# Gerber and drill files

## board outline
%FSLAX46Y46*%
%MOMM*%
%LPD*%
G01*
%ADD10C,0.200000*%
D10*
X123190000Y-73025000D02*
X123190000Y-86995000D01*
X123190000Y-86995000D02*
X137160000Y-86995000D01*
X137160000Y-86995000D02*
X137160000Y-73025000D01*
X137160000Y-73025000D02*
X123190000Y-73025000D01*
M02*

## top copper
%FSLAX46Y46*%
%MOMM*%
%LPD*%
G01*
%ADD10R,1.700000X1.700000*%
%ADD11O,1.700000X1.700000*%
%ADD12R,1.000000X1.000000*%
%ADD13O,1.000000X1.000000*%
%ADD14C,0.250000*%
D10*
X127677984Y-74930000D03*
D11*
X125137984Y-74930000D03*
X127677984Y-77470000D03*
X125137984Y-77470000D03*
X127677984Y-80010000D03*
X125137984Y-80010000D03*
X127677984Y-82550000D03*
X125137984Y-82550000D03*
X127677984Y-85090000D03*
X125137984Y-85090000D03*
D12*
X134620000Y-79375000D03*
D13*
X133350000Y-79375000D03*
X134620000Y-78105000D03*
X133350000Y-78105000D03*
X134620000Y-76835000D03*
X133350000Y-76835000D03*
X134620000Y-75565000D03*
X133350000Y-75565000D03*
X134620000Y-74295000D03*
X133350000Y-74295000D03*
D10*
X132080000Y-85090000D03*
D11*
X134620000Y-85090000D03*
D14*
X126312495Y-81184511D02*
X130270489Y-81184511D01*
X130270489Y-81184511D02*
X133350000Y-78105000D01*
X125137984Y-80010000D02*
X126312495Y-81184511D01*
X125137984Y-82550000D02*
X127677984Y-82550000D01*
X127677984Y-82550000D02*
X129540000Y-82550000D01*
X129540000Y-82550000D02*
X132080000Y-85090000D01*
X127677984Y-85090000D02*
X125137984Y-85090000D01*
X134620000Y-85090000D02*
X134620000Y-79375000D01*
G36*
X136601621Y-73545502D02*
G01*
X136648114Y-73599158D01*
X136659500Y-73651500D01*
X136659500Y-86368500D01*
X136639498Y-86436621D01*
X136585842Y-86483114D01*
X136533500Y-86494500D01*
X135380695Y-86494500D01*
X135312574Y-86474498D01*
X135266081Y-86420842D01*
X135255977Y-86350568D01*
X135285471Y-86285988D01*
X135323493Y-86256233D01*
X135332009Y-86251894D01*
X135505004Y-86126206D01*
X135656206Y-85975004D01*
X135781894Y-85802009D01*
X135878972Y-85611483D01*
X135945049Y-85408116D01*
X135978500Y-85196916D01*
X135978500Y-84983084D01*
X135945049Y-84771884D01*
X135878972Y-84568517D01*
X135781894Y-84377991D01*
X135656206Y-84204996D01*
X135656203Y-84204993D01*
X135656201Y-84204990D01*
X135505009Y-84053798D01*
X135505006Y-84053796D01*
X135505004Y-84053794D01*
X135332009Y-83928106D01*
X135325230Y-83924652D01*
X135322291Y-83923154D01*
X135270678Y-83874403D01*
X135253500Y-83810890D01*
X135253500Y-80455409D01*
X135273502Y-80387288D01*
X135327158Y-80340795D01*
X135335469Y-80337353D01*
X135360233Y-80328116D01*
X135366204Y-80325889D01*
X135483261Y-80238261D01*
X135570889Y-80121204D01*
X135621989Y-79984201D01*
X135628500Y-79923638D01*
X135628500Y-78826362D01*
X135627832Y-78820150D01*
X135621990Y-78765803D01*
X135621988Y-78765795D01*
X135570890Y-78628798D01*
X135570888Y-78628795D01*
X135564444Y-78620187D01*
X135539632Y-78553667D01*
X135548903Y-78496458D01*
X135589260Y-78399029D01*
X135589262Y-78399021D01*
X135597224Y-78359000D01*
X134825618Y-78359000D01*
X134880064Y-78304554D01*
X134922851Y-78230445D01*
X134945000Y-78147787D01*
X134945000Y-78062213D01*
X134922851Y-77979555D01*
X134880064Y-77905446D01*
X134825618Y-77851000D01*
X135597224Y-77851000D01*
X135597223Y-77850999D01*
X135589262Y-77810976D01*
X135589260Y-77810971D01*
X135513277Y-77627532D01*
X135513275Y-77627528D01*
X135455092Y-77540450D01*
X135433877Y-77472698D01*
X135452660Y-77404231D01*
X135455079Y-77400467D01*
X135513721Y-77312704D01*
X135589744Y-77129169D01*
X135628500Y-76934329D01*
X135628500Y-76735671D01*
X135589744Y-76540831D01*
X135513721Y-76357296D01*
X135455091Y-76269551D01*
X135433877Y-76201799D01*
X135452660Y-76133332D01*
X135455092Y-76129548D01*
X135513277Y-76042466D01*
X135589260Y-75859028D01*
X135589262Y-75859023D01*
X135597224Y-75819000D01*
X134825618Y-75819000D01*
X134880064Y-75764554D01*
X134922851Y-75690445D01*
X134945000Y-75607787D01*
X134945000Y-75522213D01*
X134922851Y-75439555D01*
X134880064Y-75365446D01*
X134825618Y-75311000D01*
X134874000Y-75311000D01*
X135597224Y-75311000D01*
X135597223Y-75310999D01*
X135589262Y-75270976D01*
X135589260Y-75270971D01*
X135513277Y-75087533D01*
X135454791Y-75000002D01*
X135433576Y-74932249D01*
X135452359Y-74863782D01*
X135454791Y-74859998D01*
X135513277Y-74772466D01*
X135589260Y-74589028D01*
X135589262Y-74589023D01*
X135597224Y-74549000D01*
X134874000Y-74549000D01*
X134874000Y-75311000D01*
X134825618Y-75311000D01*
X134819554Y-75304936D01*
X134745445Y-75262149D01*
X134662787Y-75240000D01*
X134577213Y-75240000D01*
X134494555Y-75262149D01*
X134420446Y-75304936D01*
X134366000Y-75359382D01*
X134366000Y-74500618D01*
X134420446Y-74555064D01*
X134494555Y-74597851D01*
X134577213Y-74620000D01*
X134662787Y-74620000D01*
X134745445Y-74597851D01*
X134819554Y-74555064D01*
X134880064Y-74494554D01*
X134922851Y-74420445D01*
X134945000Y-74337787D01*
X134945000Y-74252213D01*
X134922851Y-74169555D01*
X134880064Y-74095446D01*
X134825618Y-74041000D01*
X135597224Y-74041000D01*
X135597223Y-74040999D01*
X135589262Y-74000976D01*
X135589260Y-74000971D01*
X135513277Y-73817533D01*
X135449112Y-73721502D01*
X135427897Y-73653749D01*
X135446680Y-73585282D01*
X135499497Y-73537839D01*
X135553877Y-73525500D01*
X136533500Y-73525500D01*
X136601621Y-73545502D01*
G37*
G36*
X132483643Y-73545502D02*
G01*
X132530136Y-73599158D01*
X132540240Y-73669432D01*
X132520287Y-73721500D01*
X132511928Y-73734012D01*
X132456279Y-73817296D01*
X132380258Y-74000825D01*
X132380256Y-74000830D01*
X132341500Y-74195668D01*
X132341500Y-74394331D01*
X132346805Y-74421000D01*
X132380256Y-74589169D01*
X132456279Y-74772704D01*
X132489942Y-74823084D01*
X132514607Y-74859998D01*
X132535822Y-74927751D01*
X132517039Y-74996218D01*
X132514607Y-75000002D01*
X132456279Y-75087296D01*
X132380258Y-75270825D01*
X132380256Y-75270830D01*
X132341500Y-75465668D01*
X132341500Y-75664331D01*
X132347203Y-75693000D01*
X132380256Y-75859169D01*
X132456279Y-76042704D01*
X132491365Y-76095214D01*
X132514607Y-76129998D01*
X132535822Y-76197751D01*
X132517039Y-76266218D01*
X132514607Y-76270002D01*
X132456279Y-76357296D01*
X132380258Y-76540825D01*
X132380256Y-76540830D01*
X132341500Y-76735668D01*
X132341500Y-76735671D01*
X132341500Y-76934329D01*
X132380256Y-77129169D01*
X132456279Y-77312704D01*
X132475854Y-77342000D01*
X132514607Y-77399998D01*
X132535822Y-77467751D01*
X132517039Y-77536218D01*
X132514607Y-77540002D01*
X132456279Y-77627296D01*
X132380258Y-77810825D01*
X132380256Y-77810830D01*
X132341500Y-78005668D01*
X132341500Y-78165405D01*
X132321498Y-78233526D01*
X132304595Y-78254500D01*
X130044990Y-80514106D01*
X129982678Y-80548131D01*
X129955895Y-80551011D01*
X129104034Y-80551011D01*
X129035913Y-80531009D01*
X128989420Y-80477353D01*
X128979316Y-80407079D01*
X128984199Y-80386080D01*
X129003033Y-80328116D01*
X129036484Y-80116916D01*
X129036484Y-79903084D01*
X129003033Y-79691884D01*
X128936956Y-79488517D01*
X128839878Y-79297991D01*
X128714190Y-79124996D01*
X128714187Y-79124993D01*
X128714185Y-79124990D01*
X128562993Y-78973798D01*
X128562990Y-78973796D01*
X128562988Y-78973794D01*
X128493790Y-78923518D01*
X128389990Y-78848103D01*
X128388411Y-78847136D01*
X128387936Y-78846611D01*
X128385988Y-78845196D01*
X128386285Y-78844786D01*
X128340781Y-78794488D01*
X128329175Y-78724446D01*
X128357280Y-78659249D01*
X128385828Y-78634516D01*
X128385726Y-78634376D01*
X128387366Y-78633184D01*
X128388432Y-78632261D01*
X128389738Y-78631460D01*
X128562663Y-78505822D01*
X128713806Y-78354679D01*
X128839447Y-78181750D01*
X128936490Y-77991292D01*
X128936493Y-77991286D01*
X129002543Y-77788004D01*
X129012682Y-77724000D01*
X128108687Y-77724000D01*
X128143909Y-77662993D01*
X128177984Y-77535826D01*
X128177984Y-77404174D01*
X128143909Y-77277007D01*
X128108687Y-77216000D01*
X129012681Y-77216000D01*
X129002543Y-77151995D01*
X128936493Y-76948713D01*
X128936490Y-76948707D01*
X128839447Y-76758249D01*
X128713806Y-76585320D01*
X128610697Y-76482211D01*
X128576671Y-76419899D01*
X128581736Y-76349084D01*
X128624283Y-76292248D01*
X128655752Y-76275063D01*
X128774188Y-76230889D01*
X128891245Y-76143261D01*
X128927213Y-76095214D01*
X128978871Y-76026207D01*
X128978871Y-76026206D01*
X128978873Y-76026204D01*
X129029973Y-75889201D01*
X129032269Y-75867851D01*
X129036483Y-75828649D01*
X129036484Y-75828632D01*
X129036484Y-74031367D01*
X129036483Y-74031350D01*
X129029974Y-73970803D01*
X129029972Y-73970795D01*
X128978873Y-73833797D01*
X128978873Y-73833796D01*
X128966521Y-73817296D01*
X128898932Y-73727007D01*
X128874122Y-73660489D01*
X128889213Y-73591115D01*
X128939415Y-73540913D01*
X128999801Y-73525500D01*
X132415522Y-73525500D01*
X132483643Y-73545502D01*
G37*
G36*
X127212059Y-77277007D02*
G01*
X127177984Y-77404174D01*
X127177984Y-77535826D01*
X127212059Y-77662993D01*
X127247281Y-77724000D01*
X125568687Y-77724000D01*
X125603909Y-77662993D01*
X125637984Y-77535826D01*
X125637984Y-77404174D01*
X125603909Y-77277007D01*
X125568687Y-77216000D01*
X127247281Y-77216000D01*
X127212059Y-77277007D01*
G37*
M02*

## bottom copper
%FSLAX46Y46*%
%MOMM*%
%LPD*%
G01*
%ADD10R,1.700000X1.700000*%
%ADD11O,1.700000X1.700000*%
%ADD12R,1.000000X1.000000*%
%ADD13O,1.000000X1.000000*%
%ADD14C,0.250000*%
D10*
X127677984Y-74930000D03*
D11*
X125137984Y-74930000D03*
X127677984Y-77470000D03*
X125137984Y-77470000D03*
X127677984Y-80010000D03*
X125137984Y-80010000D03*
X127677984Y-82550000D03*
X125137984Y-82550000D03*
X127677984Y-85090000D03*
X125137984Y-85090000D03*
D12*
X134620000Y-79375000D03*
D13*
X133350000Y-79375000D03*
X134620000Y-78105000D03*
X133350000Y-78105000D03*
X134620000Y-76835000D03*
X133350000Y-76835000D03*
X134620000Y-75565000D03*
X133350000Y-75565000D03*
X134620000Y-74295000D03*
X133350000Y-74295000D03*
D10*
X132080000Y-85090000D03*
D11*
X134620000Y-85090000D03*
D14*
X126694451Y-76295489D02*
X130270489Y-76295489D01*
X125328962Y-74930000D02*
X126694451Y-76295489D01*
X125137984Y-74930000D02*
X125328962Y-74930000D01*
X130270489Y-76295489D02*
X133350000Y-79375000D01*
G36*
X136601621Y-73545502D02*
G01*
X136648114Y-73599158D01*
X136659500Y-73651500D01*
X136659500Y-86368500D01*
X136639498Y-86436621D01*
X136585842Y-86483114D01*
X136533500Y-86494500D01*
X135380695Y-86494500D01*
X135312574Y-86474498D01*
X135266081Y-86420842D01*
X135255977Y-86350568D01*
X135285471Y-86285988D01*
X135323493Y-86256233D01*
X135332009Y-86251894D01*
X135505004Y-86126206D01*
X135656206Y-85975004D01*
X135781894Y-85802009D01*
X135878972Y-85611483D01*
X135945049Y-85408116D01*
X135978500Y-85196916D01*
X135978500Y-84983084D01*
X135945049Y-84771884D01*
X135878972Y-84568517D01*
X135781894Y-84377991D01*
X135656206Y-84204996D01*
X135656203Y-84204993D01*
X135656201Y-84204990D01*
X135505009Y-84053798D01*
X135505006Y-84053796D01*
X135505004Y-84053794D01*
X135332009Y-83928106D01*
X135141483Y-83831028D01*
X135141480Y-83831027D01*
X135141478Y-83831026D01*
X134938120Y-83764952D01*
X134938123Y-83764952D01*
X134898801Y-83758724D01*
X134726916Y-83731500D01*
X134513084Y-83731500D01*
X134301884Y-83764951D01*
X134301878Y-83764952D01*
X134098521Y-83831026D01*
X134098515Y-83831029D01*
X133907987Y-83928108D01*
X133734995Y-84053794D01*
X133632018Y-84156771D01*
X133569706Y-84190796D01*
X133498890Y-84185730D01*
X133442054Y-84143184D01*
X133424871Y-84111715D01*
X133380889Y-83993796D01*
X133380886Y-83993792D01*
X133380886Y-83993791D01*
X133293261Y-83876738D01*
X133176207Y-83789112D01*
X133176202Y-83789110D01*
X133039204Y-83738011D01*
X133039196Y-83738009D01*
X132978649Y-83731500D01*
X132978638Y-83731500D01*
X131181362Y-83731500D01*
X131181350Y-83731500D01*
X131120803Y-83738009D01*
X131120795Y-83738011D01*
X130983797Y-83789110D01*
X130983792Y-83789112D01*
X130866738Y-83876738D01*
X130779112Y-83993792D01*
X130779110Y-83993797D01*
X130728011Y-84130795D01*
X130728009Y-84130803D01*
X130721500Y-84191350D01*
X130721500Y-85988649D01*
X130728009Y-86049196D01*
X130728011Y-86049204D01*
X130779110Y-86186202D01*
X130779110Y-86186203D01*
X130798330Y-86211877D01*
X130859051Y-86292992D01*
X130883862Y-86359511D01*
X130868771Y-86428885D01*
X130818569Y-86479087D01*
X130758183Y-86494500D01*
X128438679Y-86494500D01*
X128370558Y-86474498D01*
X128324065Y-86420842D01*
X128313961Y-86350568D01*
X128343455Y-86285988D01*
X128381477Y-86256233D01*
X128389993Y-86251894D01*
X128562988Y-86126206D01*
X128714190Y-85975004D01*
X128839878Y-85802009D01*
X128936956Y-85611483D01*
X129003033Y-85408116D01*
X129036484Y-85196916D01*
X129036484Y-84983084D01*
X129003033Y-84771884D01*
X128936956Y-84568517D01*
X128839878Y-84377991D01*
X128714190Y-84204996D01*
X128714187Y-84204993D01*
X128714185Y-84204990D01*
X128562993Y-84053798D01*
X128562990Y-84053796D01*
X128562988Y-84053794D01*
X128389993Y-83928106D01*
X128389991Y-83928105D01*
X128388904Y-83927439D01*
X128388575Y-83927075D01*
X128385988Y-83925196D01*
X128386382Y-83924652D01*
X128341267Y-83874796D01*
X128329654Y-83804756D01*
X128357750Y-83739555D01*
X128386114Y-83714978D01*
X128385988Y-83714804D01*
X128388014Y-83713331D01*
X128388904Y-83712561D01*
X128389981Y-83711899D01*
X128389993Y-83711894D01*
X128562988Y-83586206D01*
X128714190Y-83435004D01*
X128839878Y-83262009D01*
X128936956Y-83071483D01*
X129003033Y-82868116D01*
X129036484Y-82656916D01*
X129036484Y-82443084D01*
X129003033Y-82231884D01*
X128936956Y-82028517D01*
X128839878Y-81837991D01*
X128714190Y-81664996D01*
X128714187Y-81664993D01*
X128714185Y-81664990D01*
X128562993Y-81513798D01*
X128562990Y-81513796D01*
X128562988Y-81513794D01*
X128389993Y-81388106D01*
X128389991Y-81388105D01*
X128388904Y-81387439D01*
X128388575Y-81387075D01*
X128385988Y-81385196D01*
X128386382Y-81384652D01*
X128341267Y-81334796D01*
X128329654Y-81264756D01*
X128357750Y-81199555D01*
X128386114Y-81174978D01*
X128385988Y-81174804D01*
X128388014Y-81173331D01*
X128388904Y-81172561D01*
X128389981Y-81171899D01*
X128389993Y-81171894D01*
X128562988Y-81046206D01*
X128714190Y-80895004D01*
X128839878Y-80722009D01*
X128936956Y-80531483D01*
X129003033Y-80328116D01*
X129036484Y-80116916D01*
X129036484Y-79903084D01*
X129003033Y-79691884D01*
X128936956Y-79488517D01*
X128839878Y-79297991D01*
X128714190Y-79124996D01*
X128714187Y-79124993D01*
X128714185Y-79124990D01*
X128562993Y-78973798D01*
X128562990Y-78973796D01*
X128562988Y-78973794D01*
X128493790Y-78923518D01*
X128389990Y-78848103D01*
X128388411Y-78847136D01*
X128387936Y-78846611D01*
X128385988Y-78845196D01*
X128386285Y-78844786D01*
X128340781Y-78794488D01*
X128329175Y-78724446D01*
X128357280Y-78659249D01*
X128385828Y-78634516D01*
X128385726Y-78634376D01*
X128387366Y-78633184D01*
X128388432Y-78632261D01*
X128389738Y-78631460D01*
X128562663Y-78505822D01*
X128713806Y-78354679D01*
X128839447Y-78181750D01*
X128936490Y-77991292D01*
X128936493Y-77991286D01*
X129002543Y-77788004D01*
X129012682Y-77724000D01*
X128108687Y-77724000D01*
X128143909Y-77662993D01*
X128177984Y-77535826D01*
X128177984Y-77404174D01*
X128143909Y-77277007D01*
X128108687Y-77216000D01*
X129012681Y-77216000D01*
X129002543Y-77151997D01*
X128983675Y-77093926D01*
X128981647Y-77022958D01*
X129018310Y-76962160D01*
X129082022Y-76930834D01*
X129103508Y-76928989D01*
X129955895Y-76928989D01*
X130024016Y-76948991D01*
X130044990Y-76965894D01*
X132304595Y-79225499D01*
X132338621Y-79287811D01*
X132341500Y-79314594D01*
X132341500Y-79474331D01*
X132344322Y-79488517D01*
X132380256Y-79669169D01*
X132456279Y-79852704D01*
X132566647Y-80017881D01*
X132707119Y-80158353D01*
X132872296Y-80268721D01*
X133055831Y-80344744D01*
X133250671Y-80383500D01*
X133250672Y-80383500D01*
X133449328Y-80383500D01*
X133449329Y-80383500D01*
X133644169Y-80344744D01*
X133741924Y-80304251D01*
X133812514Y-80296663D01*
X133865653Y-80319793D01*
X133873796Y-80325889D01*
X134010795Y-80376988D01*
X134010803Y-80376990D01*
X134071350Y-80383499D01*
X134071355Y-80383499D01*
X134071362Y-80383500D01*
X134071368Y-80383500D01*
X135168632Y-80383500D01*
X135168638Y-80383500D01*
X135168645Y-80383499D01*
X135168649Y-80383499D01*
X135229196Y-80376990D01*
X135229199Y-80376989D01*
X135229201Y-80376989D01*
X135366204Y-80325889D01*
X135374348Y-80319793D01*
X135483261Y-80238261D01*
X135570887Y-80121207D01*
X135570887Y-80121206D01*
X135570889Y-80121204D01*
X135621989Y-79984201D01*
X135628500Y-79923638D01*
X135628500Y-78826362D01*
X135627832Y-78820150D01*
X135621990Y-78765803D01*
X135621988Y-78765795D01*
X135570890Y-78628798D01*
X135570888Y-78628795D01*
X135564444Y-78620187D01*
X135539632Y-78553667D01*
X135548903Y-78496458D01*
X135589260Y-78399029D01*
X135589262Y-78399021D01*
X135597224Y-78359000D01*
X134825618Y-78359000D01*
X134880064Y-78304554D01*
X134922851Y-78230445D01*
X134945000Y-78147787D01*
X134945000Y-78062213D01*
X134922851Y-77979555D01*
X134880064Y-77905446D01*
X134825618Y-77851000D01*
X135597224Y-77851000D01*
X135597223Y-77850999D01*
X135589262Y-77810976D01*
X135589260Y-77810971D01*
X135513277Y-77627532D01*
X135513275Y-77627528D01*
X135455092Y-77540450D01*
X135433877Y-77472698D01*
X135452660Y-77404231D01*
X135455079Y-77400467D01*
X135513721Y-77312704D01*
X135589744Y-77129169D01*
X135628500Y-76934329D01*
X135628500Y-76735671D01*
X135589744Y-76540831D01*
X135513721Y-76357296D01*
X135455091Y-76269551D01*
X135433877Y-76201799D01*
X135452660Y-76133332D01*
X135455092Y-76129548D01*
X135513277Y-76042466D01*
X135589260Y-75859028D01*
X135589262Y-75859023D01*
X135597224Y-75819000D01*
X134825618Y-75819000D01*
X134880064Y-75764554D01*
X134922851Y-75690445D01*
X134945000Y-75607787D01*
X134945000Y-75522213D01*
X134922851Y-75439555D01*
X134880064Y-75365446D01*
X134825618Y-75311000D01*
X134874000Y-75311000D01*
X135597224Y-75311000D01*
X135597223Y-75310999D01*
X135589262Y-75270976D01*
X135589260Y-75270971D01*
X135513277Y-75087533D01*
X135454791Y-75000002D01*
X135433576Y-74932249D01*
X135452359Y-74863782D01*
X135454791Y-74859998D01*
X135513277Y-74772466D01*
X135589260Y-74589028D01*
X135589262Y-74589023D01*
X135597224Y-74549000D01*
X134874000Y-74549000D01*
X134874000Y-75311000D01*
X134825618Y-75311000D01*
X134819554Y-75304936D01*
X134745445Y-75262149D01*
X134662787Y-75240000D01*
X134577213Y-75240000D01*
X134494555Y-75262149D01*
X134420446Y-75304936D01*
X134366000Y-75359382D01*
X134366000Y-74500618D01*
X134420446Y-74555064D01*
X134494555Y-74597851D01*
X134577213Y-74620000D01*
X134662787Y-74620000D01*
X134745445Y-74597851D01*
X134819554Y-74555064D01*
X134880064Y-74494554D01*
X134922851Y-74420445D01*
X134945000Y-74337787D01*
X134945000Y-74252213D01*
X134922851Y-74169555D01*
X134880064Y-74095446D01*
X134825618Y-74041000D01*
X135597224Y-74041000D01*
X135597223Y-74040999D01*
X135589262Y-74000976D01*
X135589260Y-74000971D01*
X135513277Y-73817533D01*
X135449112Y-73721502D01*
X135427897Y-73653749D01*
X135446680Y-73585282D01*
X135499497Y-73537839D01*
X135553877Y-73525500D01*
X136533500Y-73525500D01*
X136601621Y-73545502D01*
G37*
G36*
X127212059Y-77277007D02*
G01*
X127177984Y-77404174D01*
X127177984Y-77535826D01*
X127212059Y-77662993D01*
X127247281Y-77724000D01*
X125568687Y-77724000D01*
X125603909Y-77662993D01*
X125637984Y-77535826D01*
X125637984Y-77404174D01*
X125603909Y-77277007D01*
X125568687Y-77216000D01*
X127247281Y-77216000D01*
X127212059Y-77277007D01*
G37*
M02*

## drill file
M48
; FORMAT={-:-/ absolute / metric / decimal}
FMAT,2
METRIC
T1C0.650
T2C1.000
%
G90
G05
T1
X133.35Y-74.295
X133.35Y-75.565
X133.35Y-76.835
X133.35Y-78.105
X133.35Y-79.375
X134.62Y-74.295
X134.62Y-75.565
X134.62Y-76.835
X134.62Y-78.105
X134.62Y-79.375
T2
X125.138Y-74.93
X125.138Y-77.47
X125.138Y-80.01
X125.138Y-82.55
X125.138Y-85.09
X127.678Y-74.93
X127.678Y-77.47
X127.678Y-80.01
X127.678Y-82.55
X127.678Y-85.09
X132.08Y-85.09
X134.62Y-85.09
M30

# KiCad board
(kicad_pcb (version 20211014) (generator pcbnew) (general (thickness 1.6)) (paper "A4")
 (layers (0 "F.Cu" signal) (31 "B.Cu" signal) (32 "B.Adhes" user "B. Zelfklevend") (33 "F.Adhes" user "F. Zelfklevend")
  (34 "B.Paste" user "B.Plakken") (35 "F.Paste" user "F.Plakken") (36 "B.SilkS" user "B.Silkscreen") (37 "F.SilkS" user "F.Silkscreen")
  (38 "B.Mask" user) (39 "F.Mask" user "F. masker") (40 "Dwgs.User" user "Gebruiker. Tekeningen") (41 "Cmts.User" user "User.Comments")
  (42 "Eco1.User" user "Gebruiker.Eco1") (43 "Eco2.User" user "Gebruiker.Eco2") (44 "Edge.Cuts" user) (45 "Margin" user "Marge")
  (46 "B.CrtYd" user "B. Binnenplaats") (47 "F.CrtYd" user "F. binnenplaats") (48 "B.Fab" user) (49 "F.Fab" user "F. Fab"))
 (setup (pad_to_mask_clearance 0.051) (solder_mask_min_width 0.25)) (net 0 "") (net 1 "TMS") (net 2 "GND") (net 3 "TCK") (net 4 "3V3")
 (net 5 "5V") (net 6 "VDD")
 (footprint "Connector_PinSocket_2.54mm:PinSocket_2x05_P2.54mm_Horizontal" (layer "F.Cu") (at 127.677984 74.93)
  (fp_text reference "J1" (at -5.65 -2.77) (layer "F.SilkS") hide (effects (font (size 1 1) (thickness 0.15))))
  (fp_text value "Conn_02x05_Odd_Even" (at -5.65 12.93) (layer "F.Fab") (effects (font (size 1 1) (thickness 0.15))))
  (pad "1" thru_hole rect locked (at 0 0) (size 1.7 1.7) (drill 1) (layers *.Cu *.Mask))
  (pad "2" thru_hole oval locked (at -2.54 0) (size 1.7 1.7) (drill 1) (layers *.Cu *.Mask) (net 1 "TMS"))
  (pad "3" thru_hole oval locked (at 0 2.54) (size 1.7 1.7) (drill 1) (layers *.Cu *.Mask) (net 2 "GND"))
  (pad "4" thru_hole oval locked (at -2.54 2.54) (size 1.7 1.7) (drill 1) (layers *.Cu *.Mask) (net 2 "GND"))
  (pad "5" thru_hole oval locked (at 0 5.08) (size 1.7 1.7) (drill 1) (layers *.Cu *.Mask))
  (pad "6" thru_hole oval locked (at -2.54 5.08) (size 1.7 1.7) (drill 1) (layers *.Cu *.Mask) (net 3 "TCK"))
  (pad "7" thru_hole oval locked (at 0 7.62) (size 1.7 1.7) (drill 1) (layers *.Cu *.Mask) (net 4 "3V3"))
  (pad "8" thru_hole oval locked (at -2.54 7.62) (size 1.7 1.7) (drill 1) (layers *.Cu *.Mask) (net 4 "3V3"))
  (pad "9" thru_hole oval locked (at 0 10.16) (size 1.7 1.7) (drill 1) (layers *.Cu *.Mask) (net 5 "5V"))
  (pad "10" thru_hole oval locked (at -2.54 10.16) (size 1.7 1.7) (drill 1) (layers *.Cu *.Mask) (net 5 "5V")))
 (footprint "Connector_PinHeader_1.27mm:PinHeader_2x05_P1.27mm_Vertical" (layer "F.Cu") (at 134.62 79.375 180)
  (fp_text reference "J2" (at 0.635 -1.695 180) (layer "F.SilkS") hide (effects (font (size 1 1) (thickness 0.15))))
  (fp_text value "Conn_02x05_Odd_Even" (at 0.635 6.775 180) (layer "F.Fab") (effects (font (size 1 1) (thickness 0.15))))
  (pad "1" thru_hole rect locked (at 0 0 180) (size 1 1) (drill 0.65) (layers *.Cu *.Mask) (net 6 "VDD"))
  (pad "2" thru_hole oval locked (at 1.27 0 180) (size 1 1) (drill 0.65) (layers *.Cu *.Mask) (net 1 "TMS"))
  (pad "3" thru_hole oval locked (at 0 1.27 180) (size 1 1) (drill 0.65) (layers *.Cu *.Mask) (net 2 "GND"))
  (pad "4" thru_hole oval locked (at 1.27 1.27 180) (size 1 1) (drill 0.65) (layers *.Cu *.Mask) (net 3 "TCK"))
  (pad "5" thru_hole oval locked (at 0 2.54 180) (size 1 1) (drill 0.65) (layers *.Cu *.Mask))
  (pad "6" thru_hole oval locked (at 1.27 2.54 180) (size 1 1) (drill 0.65) (layers *.Cu *.Mask))
  (pad "7" thru_hole oval locked (at 0 3.81 180) (size 1 1) (drill 0.65) (layers *.Cu *.Mask) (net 2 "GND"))
  (pad "8" thru_hole oval locked (at 1.27 3.81 180) (size 1 1) (drill 0.65) (layers *.Cu *.Mask))
  (pad "9" thru_hole oval locked (at 0 5.08 180) (size 1 1) (drill 0.65) (layers *.Cu *.Mask) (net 2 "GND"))
  (pad "10" thru_hole oval locked (at 1.27 5.08 180) (size 1 1) (drill 0.65) (layers *.Cu *.Mask)))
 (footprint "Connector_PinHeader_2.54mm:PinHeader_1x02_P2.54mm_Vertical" (layer "F.Cu") (at 132.08 85.09 90)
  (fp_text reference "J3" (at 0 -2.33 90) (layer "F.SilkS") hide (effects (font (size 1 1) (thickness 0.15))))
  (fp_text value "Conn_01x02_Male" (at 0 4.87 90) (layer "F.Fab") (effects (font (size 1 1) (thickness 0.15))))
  (pad "1" thru_hole rect locked (at 0 0 90) (size 1.7 1.7) (drill 1) (layers *.Cu *.Mask) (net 4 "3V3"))
  (pad "2" thru_hole oval locked (at 0 2.54 90) (size 1.7 1.7) (drill 1) (layers *.Cu *.Mask) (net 6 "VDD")))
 (gr_line (start 123.19 73.025) (end 123.19 86.995) (layer "Edge.Cuts") (width 0.2))
 (gr_line (start 123.19 86.995) (end 137.16 86.995) (layer "Edge.Cuts") (width 0.2))
 (gr_line (start 137.16 86.995) (end 137.16 73.025) (layer "Edge.Cuts") (width 0.2))
 (gr_line (start 137.16 73.025) (end 123.19 73.025) (layer "Edge.Cuts") (width 0.2))
 (segment (start 126.694451 76.295489) (end 130.270489 76.295489) (width 0.25) (layer "B.Cu") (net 1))
 (segment (start 125.328962 74.93) (end 126.694451 76.295489) (width 0.25) (layer "B.Cu") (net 1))
 (segment (start 125.137984 74.93) (end 125.328962 74.93) (width 0.25) (layer "B.Cu") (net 1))
 (segment (start 130.270489 76.295489) (end 133.35 79.375) (width 0.25) (layer "B.Cu") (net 1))
 (segment (start 126.312495 81.184511) (end 130.270489 81.184511) (width 0.25) (layer "F.Cu") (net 3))
 (segment (start 130.270489 81.184511) (end 133.35 78.105) (width 0.25) (layer "F.Cu") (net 3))
 (segment (start 125.137984 80.01) (end 126.312495 81.184511) (width 0.25) (layer "F.Cu") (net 3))
 (segment (start 125.137984 82.55) (end 127.677984 82.55) (width 0.25) (layer "F.Cu") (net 4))
 (segment (start 127.677984 82.55) (end 129.54 82.55) (width 0.25) (layer "F.Cu") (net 4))
 (segment (start 129.54 82.55) (end 132.08 85.09) (width 0.25) (layer "F.Cu") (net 4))
 (segment (start 127.677984 85.09) (end 125.137984 85.09) (width 0.25) (layer "F.Cu") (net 5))
 (segment (start 134.62 85.09) (end 134.62 79.375) (width 0.25) (layer "F.Cu") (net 6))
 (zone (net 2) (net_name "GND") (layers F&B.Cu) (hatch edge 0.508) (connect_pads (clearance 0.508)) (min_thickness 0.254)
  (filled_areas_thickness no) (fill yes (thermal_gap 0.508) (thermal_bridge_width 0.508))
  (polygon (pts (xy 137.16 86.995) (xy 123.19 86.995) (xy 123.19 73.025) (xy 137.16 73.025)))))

